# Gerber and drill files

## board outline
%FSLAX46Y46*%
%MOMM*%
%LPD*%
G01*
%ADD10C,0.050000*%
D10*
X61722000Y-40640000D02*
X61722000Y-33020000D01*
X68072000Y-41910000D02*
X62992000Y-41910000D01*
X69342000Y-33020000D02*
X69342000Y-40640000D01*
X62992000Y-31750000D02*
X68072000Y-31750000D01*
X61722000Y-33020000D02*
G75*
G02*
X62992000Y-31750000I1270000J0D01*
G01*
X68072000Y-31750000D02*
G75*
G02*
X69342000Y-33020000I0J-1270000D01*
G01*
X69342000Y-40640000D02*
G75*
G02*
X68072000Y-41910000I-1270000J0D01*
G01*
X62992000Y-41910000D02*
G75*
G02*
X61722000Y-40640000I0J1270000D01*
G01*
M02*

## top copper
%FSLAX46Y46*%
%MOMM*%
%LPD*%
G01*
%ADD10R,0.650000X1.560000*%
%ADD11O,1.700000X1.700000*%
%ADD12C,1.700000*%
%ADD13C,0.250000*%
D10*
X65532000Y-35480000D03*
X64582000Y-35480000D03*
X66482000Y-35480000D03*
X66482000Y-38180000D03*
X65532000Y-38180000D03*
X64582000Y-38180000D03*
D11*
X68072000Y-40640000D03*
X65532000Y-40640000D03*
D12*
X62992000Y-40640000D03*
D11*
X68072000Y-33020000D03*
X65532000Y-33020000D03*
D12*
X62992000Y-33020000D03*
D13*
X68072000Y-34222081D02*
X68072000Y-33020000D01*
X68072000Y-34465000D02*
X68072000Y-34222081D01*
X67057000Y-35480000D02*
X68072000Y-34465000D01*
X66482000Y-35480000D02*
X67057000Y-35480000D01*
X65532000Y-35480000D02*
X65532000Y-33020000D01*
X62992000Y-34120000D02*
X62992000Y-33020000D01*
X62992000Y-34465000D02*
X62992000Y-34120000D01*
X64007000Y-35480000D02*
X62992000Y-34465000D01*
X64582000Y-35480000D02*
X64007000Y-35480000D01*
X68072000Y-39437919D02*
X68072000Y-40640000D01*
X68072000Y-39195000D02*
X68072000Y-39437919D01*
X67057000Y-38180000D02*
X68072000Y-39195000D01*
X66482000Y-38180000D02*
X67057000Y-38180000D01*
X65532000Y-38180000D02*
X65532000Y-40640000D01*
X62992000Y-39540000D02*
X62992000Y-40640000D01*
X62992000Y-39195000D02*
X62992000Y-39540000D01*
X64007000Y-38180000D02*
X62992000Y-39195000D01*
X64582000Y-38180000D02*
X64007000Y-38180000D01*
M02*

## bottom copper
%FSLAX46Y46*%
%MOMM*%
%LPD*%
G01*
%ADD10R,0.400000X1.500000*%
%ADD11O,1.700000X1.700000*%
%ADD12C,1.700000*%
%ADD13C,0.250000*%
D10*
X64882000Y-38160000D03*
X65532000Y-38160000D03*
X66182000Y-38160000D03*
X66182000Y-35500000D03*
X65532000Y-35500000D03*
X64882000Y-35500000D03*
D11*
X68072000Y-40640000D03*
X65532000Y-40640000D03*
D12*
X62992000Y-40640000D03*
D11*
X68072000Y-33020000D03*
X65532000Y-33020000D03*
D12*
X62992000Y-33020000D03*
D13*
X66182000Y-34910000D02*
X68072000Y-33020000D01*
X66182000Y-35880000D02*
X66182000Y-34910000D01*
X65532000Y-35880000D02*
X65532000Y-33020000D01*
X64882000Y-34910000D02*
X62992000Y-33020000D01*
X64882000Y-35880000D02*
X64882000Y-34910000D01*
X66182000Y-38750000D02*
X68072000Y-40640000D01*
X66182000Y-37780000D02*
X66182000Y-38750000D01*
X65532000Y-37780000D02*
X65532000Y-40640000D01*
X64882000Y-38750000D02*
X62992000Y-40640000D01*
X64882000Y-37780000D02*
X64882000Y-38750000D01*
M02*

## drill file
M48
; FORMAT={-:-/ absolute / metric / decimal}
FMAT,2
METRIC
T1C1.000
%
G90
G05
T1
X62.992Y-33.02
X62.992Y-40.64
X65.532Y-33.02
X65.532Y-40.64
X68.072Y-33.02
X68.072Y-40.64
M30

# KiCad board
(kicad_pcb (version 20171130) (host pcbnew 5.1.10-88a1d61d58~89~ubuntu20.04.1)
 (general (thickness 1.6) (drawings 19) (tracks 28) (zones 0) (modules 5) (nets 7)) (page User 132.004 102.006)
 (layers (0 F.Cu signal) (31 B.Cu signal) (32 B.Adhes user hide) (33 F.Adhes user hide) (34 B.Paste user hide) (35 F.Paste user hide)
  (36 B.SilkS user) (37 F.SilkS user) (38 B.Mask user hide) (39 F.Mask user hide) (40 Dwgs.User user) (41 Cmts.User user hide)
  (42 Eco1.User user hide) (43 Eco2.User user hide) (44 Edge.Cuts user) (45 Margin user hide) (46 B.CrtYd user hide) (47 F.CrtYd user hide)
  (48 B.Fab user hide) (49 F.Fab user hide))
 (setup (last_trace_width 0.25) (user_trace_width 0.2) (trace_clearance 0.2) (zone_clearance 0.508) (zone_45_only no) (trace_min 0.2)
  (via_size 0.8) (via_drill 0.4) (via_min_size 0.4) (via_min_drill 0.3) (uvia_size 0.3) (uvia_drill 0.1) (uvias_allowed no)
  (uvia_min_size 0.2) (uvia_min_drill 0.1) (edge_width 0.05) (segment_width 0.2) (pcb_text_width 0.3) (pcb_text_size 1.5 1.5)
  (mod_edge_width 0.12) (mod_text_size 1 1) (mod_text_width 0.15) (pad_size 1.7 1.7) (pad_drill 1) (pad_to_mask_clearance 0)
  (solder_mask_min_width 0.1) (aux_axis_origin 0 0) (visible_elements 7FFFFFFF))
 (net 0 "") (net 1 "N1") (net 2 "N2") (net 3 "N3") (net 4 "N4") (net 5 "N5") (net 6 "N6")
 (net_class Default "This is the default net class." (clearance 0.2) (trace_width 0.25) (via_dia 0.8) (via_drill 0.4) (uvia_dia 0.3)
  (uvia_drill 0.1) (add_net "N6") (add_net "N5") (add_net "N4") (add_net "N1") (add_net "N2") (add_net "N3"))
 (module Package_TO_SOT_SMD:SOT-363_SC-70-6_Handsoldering (layer B.Cu) (at 65.532 36.83 270)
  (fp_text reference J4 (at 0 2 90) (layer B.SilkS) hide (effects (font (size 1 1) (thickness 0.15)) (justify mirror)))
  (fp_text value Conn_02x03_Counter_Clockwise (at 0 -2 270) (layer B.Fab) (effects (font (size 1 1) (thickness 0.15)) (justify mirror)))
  (pad 6 smd rect (at 1.33 0.65 270) (size 1.5 0.4) (layers B.Cu B.Paste B.Mask) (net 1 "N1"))
  (pad 5 smd rect (at 1.33 0 270) (size 1.5 0.4) (layers B.Cu B.Paste B.Mask) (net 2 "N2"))
  (pad 4 smd rect (at 1.33 -0.65 270) (size 1.5 0.4) (layers B.Cu B.Paste B.Mask) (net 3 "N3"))
  (pad 3 smd rect (at -1.33 -0.65 270) (size 1.5 0.4) (layers B.Cu B.Paste B.Mask) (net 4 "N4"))
  (pad 2 smd rect (at -1.33 0 270) (size 1.5 0.4) (layers B.Cu B.Paste B.Mask) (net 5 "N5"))
  (pad 1 smd rect (at -1.33 0.65 270) (size 1.5 0.4) (layers B.Cu B.Paste B.Mask) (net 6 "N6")))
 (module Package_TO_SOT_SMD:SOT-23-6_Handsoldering (layer F.Cu) (at 65.532 36.83 90)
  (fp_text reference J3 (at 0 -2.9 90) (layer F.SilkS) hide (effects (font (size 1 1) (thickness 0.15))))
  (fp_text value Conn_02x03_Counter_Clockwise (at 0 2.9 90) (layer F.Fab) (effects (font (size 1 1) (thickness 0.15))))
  (pad 5 smd rect (at 1.35 0 90) (size 1.56 0.65) (layers F.Cu F.Paste F.Mask) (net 5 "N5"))
  (pad 6 smd rect (at 1.35 -0.95 90) (size 1.56 0.65) (layers F.Cu F.Paste F.Mask) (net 6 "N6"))
  (pad 4 smd rect (at 1.35 0.95 90) (size 1.56 0.65) (layers F.Cu F.Paste F.Mask) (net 4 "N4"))
  (pad 3 smd rect (at -1.35 0.95 90) (size 1.56 0.65) (layers F.Cu F.Paste F.Mask) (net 3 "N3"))
  (pad 2 smd rect (at -1.35 0 90) (size 1.56 0.65) (layers F.Cu F.Paste F.Mask) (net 2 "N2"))
  (pad 1 smd rect (at -1.35 -0.95 90) (size 1.56 0.65) (layers F.Cu F.Paste F.Mask) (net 1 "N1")))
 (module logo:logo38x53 (layer B.Cu) (at 53.4797 34.2646 180)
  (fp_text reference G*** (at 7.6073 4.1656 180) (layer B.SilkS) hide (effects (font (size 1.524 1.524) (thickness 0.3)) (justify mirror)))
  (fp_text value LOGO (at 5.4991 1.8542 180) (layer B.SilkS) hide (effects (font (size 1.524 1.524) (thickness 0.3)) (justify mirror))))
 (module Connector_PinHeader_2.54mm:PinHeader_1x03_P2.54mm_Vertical (layer F.Cu) (at 62.992 40.64 90)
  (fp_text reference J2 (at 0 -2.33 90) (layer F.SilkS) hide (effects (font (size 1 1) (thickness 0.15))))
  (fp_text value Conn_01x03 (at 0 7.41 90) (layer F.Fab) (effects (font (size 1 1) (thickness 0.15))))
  (pad 3 thru_hole oval (at 0 5.08 90) (size 1.7 1.7) (drill 1) (layers *.Cu *.Mask) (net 3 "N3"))
  (pad 2 thru_hole oval (at 0 2.54 90) (size 1.7 1.7) (drill 1) (layers *.Cu *.Mask) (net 2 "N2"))
  (pad 1 thru_hole circle (at 0 0 90) (size 1.7 1.7) (drill 1) (layers *.Cu *.Mask) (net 1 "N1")))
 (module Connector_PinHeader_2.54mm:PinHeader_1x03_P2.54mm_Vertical (layer F.Cu) (at 62.992 33.02 90)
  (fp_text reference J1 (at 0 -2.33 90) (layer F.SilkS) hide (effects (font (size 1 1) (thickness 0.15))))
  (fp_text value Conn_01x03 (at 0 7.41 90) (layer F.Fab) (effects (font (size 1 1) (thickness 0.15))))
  (pad 3 thru_hole oval (at 0 5.08 90) (size 1.7 1.7) (drill 1) (layers *.Cu *.Mask) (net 4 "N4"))
  (pad 2 thru_hole oval (at 0 2.54 90) (size 1.7 1.7) (drill 1) (layers *.Cu *.Mask) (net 5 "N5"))
  (pad 1 thru_hole circle (at 0 0 90) (size 1.7 1.7) (drill 1) (layers *.Cu *.Mask) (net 6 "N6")))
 (gr_line (start 61.722 40.64) (end 61.722 33.02) (layer Edge.Cuts) (width 0.05))
 (gr_line (start 68.072 41.91) (end 62.992 41.91) (layer Edge.Cuts) (width 0.05))
 (gr_line (start 69.342 33.02) (end 69.342 40.64) (layer Edge.Cuts) (width 0.05))
 (gr_line (start 62.992 31.75) (end 68.072 31.75) (layer Edge.Cuts) (width 0.05))
 (gr_arc (start 62.992 33.02) (end 62.992 31.75) (angle -90) (layer Edge.Cuts) (width 0.05))
 (gr_arc (start 68.072 33.02) (end 69.342 33.02) (angle -90) (layer Edge.Cuts) (width 0.05))
 (gr_arc (start 68.072 40.64) (end 68.072 41.91) (angle -90) (layer Edge.Cuts) (width 0.05))
 (gr_arc (start 62.992 40.64) (end 61.722 40.64) (angle -90) (layer Edge.Cuts) (width 0.05))
 (segment (start 68.072 34.222081) (end 68.072 33.02) (width 0.25) (layer F.Cu) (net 4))
 (segment (start 68.072 34.465) (end 68.072 34.222081) (width 0.25) (layer F.Cu) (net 4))
 (segment (start 67.057 35.48) (end 68.072 34.465) (width 0.25) (layer F.Cu) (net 4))
 (segment (start 66.482 35.48) (end 67.057 35.48) (width 0.25) (layer F.Cu) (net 4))
 (segment (start 66.182 34.91) (end 68.072 33.02) (width 0.25) (layer B.Cu) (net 4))
 (segment (start 66.182 35.88) (end 66.182 34.91) (width 0.25) (layer B.Cu) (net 4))
 (segment (start 65.532 35.48) (end 65.532 33.02) (width 0.25) (layer F.Cu) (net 5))
 (segment (start 65.532 35.88) (end 65.532 33.02) (width 0.25) (layer B.Cu) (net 5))
 (segment (start 62.992 34.12) (end 62.992 33.02) (width 0.25) (layer F.Cu) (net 6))
 (segment (start 62.992 34.465) (end 62.992 34.12) (width 0.25) (layer F.Cu) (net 6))
 (segment (start 64.007 35.48) (end 62.992 34.465) (width 0.25) (layer F.Cu) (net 6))
 (segment (start 64.582 35.48) (end 64.007 35.48) (width 0.25) (layer F.Cu) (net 6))
 (segment (start 64.882 34.91) (end 62.992 33.02) (width 0.25) (layer B.Cu) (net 6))
 (segment (start 64.882 35.88) (end 64.882 34.91) (width 0.25) (layer B.Cu) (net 6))
 (segment (start 68.072 39.437919) (end 68.072 40.64) (width 0.25) (layer F.Cu) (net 3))
 (segment (start 68.072 39.195) (end 68.072 39.437919) (width 0.25) (layer F.Cu) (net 3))
 (segment (start 67.057 38.18) (end 68.072 39.195) (width 0.25) (layer F.Cu) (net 3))
 (segment (start 66.482 38.18) (end 67.057 38.18) (width 0.25) (layer F.Cu) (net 3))
 (segment (start 66.182 38.75) (end 68.072 40.64) (width 0.25) (layer B.Cu) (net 3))
 (segment (start 66.182 37.78) (end 66.182 38.75) (width 0.25) (layer B.Cu) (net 3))
 (segment (start 65.532 38.18) (end 65.532 40.64) (width 0.25) (layer F.Cu) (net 2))
 (segment (start 65.532 37.78) (end 65.532 40.64) (width 0.25) (layer B.Cu) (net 2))
 (segment (start 62.992 39.54) (end 62.992 40.64) (width 0.25) (layer F.Cu) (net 1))
 (segment (start 62.992 39.195) (end 62.992 39.54) (width 0.25) (layer F.Cu) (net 1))
 (segment (start 64.007 38.18) (end 62.992 39.195) (width 0.25) (layer F.Cu) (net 1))
 (segment (start 64.582 38.18) (end 64.007 38.18) (width 0.25) (layer F.Cu) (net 1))
 (segment (start 64.882 38.75) (end 62.992 40.64) (width 0.25) (layer B.Cu) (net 1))
 (segment (start 64.882 37.78) (end 64.882 38.75) (width 0.25) (layer B.Cu) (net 1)))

